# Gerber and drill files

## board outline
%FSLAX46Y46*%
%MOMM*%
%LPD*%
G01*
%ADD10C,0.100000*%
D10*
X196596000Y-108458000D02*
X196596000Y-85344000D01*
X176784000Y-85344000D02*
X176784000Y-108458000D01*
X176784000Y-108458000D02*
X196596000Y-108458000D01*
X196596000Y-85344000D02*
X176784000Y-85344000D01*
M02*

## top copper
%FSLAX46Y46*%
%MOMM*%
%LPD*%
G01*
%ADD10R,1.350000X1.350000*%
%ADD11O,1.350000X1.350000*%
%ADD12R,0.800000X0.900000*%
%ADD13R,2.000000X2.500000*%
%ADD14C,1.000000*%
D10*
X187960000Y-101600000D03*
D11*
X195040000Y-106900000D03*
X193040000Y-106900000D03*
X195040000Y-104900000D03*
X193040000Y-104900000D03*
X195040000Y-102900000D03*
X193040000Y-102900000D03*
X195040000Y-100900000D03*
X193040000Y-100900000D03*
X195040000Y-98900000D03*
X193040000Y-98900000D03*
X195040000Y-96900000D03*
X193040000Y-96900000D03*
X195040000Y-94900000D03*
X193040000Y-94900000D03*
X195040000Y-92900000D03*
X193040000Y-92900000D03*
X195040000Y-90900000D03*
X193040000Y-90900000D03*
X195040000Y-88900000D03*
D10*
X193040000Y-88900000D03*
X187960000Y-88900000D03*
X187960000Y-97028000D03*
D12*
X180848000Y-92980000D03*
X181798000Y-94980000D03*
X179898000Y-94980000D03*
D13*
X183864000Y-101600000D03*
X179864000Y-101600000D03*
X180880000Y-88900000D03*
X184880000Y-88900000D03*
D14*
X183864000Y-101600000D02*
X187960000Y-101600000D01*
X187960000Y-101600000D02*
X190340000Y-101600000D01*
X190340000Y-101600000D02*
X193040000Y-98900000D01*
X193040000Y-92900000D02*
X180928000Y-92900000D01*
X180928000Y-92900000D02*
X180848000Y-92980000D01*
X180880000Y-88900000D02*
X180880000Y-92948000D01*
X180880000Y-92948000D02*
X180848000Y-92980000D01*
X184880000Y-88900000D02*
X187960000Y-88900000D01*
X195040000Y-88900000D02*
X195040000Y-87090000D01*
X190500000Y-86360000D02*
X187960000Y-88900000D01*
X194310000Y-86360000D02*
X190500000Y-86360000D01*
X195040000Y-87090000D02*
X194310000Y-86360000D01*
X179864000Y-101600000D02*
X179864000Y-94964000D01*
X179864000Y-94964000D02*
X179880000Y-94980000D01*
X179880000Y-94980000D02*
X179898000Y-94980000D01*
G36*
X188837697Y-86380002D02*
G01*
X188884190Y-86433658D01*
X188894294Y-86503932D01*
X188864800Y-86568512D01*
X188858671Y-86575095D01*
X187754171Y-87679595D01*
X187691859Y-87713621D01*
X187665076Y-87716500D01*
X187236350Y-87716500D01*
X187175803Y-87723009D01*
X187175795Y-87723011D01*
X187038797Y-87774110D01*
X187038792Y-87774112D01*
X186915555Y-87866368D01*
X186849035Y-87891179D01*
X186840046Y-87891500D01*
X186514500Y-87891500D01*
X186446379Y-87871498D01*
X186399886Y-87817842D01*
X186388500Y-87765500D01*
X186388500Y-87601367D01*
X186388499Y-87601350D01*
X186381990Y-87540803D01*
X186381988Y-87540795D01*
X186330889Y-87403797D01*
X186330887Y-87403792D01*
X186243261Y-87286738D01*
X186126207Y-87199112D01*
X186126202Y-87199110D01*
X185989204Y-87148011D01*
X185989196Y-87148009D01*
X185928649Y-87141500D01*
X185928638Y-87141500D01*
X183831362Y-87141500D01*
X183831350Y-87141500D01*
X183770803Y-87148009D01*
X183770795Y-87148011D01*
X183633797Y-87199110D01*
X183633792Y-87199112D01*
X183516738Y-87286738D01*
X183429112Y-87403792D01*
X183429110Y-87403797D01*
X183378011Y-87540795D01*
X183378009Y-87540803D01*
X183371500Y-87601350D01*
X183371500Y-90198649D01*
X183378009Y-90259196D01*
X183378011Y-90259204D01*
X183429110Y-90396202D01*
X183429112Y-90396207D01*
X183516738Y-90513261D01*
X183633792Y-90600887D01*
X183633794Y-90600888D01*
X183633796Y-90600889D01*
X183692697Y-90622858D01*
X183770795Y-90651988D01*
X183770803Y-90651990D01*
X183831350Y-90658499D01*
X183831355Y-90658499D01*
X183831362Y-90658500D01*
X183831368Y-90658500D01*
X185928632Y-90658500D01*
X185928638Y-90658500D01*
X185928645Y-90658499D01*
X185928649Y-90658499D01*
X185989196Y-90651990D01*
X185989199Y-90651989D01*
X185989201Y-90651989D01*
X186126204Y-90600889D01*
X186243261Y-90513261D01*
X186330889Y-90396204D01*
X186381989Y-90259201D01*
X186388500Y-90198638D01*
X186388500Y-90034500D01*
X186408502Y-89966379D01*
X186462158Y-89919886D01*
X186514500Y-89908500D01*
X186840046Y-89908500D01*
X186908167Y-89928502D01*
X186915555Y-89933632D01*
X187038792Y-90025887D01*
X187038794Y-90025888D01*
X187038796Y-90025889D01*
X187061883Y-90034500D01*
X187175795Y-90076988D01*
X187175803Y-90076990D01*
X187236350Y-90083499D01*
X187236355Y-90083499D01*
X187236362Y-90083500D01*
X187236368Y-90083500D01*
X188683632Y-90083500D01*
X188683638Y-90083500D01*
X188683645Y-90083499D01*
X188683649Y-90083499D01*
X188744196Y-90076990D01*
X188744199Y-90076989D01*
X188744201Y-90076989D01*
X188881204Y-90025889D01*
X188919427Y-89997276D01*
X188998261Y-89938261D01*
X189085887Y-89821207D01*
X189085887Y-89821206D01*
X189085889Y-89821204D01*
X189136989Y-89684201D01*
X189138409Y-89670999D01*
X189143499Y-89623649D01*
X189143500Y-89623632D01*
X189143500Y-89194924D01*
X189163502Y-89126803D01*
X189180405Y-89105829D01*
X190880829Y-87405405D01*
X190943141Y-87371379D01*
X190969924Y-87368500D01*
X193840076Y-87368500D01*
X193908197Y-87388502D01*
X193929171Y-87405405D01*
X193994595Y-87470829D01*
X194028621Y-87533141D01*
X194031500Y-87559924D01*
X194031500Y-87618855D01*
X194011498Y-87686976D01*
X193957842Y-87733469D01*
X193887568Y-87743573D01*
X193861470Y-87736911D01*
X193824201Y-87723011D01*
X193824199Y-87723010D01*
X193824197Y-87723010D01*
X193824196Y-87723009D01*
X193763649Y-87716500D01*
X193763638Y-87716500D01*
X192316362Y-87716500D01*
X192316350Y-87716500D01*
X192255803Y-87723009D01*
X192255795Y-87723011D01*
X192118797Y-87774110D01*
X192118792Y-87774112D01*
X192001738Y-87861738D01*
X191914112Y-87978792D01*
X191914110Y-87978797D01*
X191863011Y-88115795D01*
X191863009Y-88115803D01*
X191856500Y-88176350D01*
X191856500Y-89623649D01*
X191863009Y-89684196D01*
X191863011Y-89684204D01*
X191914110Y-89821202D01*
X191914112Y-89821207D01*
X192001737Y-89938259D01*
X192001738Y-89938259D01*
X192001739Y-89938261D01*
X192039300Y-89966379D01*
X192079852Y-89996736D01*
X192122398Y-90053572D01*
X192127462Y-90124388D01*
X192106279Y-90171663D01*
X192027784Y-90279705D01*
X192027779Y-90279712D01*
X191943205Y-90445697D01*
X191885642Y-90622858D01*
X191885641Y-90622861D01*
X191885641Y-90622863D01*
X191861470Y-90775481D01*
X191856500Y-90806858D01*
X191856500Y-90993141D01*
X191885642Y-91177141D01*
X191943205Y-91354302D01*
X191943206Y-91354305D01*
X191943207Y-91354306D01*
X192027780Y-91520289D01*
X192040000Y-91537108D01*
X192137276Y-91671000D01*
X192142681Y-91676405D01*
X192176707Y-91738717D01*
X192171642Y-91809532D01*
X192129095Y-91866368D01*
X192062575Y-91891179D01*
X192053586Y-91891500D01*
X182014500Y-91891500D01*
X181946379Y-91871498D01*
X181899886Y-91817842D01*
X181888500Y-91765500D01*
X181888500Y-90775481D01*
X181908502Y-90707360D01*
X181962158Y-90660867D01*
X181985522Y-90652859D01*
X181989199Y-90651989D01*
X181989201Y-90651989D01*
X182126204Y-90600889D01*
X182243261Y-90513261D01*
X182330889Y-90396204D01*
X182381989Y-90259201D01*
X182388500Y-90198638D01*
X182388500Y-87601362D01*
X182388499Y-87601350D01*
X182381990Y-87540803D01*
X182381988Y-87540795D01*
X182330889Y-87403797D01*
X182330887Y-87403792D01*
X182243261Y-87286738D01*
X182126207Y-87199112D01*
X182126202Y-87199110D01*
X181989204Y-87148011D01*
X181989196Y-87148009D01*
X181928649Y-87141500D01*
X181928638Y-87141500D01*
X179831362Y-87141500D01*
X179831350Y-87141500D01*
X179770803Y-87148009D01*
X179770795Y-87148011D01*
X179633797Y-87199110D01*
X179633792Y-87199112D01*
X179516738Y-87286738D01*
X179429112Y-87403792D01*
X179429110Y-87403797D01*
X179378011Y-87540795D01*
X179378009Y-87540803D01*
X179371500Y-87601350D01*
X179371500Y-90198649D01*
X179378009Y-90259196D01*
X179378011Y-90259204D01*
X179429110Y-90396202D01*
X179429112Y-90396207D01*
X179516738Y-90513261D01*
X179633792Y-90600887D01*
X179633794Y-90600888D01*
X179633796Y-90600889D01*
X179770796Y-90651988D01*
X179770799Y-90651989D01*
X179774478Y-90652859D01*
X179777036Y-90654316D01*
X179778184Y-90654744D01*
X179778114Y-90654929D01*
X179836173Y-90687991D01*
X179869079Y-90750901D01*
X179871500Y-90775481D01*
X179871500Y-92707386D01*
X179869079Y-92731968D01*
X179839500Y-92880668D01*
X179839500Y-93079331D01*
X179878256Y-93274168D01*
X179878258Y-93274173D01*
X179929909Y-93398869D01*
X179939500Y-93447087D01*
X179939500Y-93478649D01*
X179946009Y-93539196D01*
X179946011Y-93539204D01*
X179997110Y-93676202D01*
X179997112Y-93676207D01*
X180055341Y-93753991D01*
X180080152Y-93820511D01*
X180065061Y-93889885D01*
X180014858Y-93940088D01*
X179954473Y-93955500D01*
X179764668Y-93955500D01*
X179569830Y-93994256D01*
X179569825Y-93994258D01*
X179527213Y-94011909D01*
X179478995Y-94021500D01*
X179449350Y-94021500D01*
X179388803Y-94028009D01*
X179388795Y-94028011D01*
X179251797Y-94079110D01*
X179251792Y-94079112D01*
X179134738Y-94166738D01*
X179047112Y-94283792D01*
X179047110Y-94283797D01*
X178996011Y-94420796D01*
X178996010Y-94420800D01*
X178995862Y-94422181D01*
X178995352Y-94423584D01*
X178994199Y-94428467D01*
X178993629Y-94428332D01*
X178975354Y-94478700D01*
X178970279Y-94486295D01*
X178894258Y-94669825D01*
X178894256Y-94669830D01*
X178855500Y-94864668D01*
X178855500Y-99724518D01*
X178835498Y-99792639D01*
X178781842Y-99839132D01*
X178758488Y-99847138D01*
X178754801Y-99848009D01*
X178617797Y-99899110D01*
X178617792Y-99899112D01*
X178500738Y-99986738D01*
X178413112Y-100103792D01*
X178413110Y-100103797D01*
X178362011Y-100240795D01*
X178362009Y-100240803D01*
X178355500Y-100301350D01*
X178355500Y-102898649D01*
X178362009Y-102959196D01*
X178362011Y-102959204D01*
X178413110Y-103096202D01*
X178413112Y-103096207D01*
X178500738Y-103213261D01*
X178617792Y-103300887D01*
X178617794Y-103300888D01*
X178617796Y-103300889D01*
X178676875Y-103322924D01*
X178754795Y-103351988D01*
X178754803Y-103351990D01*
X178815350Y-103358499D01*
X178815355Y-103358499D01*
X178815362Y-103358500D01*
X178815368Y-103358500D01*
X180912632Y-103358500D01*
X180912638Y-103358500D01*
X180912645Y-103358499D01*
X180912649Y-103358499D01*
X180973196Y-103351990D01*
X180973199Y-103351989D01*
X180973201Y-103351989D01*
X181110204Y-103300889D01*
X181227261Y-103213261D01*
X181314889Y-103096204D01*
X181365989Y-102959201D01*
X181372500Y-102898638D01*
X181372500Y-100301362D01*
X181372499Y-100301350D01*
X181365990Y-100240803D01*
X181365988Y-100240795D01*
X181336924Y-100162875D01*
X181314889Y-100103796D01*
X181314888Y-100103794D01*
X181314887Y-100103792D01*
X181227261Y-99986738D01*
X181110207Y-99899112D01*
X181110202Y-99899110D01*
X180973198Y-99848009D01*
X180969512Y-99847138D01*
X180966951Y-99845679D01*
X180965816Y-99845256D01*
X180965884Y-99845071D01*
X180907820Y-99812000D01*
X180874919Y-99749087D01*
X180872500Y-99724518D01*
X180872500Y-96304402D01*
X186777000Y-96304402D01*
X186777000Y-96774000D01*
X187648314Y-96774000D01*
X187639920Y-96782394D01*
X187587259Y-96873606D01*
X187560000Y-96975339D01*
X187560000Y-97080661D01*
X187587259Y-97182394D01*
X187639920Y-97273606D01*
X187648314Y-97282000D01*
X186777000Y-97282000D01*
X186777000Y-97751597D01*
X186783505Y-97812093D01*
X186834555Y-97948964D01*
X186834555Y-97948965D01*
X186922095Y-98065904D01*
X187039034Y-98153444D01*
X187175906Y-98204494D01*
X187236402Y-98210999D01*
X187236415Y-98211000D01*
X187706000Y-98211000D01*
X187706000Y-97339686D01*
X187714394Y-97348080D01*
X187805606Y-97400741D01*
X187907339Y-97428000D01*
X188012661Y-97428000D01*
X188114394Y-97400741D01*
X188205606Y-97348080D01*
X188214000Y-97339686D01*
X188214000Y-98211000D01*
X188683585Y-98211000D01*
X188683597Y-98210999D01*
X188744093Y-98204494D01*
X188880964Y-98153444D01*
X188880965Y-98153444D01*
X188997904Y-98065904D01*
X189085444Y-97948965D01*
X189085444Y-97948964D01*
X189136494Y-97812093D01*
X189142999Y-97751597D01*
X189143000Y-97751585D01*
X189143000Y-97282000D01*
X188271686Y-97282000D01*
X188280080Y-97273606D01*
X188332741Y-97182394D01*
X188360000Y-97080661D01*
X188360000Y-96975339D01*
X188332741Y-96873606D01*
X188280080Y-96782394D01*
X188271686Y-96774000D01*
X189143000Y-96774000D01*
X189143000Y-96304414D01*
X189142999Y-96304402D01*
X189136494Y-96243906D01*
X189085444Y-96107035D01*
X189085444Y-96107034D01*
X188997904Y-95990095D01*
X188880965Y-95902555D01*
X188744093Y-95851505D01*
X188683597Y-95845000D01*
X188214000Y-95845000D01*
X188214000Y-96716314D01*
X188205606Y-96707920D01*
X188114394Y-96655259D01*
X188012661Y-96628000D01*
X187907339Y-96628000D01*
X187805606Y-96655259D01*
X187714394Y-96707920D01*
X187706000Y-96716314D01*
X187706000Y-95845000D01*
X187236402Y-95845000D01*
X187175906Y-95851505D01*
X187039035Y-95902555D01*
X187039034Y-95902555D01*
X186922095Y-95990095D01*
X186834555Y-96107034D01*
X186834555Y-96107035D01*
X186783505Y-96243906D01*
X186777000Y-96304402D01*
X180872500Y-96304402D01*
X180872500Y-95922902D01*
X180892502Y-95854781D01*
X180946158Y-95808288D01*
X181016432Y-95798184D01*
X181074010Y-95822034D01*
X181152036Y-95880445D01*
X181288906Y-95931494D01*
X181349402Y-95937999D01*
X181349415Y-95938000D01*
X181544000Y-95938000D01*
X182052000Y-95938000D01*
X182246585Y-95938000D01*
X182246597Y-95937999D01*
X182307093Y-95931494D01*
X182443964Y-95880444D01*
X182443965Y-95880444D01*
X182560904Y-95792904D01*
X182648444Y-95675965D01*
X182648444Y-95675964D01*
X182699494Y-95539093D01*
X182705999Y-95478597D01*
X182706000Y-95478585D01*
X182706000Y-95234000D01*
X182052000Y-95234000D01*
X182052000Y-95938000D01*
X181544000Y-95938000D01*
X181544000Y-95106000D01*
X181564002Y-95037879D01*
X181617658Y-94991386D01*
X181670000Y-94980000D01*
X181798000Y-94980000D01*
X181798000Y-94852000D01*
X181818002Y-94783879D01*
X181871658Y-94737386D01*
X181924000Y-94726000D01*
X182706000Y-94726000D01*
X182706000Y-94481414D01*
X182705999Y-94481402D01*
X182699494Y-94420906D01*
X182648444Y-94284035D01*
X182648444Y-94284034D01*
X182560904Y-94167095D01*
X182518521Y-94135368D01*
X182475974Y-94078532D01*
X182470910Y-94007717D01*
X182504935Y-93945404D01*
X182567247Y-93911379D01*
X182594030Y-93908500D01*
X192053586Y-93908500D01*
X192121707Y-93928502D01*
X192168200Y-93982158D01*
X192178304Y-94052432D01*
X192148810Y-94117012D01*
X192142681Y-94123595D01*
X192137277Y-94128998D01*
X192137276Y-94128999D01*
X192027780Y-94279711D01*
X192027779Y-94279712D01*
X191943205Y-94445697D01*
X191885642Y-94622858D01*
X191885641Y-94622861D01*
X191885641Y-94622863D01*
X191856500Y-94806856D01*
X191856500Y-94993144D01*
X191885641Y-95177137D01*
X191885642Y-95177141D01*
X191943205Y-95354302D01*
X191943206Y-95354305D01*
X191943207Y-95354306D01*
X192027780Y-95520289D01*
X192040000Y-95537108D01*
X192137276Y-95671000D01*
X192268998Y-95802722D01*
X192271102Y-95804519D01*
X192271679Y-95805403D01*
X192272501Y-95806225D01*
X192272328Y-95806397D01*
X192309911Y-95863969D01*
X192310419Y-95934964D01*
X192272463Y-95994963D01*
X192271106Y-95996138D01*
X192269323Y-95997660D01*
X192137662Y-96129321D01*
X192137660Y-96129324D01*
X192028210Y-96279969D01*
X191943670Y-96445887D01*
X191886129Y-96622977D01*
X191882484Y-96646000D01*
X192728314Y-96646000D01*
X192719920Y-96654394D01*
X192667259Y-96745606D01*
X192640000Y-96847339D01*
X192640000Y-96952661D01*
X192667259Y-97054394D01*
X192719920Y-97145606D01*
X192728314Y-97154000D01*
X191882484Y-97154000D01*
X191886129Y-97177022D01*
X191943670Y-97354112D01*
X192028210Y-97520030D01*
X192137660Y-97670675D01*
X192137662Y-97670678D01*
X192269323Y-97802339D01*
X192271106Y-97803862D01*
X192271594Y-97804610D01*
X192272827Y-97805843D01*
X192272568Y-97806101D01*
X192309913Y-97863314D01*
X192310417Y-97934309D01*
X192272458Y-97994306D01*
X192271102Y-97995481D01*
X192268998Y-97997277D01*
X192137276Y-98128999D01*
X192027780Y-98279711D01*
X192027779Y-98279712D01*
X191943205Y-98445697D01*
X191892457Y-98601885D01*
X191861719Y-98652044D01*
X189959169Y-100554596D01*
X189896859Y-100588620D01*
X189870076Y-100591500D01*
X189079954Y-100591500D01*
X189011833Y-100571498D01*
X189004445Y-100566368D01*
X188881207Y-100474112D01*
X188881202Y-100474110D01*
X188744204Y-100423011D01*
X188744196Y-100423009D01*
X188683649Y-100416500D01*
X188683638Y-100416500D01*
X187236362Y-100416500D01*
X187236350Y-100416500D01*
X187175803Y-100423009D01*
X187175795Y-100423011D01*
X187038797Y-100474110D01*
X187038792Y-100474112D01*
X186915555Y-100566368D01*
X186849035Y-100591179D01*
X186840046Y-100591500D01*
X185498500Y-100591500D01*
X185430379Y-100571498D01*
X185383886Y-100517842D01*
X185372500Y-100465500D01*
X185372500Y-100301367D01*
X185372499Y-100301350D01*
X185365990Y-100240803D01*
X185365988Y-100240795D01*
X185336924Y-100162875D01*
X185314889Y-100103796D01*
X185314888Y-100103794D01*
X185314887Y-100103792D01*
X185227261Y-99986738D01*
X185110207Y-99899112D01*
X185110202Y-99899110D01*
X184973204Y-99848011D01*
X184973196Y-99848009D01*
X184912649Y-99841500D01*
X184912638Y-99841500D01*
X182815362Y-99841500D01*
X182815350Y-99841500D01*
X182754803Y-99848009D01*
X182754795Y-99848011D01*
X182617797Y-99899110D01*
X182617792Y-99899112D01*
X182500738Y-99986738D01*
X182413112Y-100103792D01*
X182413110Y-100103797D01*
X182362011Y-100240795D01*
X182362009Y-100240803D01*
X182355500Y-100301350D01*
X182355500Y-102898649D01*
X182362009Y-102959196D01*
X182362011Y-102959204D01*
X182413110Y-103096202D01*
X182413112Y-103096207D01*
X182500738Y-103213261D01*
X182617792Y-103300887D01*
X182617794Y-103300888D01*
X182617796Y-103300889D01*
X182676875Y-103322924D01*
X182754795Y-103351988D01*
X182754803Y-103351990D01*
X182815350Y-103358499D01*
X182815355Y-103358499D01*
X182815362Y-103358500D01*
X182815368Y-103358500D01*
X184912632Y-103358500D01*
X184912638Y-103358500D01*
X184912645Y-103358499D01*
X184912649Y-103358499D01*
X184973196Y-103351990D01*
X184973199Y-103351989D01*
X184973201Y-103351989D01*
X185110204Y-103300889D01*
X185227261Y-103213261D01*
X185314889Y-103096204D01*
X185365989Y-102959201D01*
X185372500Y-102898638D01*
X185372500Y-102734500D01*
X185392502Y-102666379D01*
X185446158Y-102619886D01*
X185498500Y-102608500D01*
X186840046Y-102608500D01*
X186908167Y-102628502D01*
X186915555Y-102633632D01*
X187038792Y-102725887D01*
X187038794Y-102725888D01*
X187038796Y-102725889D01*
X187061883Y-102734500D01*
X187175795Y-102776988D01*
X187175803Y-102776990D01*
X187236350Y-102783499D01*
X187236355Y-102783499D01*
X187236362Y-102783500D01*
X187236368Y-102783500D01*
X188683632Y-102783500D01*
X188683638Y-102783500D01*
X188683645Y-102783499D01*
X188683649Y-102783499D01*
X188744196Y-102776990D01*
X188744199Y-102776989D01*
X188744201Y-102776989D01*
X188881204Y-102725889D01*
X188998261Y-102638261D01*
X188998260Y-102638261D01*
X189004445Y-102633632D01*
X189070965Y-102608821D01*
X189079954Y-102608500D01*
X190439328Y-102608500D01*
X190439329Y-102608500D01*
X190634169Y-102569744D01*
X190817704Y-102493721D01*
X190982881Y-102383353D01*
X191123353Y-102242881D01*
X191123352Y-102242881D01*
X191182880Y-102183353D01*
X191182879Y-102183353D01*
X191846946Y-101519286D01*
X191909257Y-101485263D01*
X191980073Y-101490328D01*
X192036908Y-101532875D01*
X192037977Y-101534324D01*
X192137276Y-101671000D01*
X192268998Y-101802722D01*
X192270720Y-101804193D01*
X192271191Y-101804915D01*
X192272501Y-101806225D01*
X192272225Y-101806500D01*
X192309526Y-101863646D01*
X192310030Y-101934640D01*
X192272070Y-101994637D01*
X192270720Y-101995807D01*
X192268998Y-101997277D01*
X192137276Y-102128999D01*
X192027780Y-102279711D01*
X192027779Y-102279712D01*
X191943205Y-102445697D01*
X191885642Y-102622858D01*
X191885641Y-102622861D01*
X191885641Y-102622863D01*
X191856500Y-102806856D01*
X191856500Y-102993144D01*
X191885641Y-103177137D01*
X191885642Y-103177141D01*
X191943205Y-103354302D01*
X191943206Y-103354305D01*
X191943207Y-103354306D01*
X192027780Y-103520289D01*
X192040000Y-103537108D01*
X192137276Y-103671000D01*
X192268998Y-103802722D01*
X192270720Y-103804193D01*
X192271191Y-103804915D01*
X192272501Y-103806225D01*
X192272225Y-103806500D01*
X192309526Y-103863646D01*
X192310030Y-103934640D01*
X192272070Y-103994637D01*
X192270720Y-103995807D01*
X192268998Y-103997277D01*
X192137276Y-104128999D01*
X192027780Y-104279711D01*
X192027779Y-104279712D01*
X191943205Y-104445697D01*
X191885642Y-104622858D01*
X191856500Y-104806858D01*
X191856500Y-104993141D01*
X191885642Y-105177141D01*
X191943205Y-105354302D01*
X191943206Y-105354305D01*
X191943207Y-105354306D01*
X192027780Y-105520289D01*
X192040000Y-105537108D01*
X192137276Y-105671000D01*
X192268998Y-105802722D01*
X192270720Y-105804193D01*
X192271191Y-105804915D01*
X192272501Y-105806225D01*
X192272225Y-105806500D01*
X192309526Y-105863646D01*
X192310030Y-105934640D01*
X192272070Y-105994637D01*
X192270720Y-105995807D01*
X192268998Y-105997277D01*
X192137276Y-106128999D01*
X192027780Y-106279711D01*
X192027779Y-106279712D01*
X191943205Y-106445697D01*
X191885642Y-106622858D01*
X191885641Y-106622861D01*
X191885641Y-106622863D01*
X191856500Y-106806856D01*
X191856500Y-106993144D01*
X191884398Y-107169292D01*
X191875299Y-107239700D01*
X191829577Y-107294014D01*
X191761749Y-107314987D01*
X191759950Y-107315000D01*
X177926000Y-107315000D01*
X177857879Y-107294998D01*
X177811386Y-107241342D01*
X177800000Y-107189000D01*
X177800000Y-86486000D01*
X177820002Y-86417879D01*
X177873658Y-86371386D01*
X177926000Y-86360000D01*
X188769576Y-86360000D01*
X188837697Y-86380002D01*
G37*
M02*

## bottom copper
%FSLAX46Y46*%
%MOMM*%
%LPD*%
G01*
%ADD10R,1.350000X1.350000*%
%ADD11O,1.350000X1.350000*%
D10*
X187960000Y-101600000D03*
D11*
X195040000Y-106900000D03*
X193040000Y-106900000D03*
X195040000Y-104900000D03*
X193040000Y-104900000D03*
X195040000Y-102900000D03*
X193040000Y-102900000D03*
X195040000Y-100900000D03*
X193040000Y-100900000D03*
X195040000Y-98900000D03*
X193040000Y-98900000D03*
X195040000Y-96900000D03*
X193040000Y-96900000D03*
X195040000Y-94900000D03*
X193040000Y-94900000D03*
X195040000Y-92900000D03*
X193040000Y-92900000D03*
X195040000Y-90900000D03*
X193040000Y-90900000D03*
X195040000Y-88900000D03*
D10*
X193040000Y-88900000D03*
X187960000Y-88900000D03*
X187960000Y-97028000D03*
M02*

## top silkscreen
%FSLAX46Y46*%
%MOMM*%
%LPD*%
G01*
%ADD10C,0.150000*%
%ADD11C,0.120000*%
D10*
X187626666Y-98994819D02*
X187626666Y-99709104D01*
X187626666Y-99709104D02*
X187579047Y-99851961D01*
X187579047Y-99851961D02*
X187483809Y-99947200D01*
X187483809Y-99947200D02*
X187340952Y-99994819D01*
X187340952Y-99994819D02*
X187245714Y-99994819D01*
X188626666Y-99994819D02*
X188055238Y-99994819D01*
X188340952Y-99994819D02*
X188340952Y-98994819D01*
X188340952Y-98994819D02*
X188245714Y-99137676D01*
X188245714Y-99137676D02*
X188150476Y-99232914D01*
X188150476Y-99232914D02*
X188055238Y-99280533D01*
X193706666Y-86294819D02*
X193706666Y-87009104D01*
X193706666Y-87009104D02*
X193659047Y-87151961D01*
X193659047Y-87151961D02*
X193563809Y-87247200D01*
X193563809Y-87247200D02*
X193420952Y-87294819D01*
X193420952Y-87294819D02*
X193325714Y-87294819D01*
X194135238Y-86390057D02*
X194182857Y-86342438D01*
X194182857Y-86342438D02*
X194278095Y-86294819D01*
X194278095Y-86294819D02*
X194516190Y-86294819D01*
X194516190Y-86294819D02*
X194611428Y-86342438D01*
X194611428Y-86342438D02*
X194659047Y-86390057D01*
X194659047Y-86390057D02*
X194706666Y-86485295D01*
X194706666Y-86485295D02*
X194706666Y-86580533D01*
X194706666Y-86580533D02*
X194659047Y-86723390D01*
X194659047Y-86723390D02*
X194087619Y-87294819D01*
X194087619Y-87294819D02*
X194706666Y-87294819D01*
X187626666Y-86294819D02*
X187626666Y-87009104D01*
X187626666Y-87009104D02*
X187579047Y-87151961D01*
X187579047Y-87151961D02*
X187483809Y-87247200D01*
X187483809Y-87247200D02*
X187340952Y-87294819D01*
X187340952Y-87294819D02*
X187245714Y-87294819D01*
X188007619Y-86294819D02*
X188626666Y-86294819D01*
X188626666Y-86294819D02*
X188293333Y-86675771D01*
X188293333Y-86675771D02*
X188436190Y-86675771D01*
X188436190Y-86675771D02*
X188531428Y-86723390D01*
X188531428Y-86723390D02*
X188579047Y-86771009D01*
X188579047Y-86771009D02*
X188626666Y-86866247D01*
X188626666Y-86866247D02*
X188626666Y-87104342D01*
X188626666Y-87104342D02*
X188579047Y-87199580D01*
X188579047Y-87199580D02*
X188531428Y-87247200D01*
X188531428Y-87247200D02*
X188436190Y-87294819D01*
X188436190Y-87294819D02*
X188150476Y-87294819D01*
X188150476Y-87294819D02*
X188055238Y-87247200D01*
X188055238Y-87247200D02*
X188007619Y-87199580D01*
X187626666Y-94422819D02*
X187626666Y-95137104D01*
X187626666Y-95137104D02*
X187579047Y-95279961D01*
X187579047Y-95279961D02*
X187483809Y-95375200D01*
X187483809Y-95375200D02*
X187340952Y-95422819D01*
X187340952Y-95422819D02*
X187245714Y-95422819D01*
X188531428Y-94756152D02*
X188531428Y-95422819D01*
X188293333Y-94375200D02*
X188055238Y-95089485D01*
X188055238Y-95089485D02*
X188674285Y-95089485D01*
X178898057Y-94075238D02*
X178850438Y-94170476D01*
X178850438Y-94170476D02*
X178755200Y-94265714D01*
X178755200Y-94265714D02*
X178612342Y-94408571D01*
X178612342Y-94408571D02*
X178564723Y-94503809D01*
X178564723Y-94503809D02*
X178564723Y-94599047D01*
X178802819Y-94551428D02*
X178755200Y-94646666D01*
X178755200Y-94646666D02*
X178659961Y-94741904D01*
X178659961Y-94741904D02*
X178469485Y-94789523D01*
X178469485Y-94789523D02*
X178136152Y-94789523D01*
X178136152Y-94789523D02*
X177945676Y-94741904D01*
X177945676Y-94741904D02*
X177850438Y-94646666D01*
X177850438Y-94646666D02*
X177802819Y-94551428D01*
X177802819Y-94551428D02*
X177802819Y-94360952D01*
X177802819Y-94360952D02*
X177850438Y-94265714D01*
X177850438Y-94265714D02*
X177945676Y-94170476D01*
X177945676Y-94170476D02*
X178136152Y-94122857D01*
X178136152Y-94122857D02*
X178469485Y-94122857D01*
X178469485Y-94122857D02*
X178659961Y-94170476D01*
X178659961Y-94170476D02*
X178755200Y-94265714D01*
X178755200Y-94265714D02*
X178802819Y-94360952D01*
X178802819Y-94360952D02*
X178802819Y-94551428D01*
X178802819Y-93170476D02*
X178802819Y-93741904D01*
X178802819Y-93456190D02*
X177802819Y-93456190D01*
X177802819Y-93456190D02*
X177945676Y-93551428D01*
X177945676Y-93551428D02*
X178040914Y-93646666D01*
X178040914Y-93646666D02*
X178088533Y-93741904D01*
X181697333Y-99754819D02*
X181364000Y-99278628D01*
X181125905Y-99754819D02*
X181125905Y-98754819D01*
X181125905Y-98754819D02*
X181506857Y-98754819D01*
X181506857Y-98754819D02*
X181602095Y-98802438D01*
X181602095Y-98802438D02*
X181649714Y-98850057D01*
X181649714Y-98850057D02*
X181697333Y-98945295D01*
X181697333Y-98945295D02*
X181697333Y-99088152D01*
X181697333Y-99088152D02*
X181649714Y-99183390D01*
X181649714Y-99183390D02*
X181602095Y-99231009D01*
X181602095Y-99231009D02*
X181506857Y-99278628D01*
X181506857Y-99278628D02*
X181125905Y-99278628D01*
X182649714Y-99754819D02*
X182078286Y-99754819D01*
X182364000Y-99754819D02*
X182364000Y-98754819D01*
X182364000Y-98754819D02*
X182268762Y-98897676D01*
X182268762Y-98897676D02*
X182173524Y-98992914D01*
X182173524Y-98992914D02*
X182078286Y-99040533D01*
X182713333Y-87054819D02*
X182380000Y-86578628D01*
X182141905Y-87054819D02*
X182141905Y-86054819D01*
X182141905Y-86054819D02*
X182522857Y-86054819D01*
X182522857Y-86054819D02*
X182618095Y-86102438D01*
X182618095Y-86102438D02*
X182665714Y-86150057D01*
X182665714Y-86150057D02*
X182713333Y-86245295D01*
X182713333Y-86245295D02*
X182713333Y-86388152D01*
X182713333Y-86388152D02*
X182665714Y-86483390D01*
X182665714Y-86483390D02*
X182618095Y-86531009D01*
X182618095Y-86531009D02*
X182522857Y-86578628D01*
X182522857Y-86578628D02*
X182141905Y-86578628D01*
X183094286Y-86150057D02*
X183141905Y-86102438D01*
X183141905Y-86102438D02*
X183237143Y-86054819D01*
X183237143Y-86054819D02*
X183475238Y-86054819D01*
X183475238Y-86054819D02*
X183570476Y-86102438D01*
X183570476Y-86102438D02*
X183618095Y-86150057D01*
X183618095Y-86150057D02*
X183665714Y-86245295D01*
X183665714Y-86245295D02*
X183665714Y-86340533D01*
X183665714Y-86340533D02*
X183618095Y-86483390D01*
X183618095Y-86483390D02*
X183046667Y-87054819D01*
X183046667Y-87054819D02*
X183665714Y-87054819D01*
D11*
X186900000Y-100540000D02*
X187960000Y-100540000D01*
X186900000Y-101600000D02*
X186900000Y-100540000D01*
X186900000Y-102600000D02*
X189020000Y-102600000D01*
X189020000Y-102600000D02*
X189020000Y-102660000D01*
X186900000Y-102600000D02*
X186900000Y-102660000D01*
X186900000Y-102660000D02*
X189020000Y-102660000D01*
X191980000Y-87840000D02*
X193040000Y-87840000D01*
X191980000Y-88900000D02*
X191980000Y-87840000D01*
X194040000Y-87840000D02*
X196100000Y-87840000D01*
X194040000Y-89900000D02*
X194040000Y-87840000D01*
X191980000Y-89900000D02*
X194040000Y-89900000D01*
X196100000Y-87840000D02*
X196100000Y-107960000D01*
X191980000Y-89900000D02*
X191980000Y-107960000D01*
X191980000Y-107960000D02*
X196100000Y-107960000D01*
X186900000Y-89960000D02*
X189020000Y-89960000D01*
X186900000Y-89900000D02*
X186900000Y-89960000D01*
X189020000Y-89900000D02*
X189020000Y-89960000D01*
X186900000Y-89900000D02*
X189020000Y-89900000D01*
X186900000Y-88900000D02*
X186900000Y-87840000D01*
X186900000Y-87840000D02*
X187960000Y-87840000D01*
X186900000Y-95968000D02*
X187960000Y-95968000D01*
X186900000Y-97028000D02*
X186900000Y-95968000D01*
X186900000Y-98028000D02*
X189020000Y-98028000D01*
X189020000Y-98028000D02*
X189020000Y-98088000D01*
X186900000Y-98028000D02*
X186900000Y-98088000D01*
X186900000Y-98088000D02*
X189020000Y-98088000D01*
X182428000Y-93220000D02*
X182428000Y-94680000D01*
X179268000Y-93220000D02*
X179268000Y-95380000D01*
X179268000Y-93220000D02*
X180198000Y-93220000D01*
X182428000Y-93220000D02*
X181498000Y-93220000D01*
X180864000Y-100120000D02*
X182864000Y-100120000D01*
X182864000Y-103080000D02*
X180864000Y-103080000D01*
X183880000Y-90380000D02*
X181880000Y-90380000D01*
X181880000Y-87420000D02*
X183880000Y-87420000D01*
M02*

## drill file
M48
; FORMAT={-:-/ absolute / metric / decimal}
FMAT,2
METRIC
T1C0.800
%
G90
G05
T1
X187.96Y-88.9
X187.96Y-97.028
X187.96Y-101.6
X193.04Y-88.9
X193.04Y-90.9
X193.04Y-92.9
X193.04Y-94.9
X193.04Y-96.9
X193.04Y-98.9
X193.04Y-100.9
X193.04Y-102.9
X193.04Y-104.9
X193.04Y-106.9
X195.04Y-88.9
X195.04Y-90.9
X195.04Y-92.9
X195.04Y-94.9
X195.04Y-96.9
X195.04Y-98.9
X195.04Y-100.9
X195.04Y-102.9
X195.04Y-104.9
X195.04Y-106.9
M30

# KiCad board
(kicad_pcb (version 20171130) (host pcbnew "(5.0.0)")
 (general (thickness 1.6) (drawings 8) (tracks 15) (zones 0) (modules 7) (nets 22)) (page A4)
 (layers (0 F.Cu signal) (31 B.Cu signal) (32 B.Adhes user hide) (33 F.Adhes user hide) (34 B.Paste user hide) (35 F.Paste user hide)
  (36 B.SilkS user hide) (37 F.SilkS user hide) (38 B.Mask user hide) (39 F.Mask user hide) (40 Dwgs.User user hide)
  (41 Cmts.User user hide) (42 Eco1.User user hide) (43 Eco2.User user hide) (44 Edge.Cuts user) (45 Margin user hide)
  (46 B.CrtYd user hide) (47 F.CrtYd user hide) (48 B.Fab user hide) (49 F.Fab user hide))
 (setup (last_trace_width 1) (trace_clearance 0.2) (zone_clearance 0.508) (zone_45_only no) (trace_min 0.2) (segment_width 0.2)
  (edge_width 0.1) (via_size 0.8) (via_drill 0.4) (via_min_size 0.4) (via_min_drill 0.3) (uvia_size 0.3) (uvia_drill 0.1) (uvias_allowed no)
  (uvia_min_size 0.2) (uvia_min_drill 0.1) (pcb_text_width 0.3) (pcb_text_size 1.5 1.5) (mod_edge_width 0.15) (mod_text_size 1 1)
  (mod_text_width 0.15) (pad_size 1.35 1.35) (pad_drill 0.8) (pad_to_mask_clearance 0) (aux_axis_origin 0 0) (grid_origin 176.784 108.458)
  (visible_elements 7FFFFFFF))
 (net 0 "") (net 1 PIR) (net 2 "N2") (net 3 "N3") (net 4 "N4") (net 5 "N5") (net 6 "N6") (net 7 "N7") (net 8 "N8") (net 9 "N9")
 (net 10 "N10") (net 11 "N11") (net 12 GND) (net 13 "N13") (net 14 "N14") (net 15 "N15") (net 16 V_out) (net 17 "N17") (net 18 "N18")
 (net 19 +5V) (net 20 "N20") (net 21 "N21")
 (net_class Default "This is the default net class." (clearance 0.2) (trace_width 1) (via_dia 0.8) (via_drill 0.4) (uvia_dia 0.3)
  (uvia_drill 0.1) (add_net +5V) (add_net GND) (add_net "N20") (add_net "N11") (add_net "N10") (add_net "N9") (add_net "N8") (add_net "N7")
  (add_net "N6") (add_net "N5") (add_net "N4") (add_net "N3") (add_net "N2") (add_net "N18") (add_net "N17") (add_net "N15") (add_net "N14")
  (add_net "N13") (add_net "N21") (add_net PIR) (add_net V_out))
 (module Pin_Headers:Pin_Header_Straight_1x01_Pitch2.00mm (layer F.Cu) (at 187.96 101.6)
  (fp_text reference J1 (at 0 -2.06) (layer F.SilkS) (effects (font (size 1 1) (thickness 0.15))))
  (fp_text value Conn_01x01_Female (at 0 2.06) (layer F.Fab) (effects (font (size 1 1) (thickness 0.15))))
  (fp_line (start -1.06 -1.06) (end 0 -1.06) (layer F.SilkS) (width 0.12))
  (fp_line (start -1.06 0) (end -1.06 -1.06) (layer F.SilkS) (width 0.12))
  (fp_line (start -1.06 1) (end 1.06 1) (layer F.SilkS) (width 0.12))
  (fp_line (start 1.06 1) (end 1.06 1.06) (layer F.SilkS) (width 0.12))
  (fp_line (start -1.06 1) (end -1.06 1.06) (layer F.SilkS) (width 0.12))
  (fp_line (start -1.06 1.06) (end 1.06 1.06) (layer F.SilkS) (width 0.12))
  (pad 1 thru_hole rect (at 0 0) (size 1.35 1.35) (drill 0.8) (layers *.Cu *.Mask) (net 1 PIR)))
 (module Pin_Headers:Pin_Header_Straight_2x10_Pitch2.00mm (layer F.Cu) (at 193.04 88.9)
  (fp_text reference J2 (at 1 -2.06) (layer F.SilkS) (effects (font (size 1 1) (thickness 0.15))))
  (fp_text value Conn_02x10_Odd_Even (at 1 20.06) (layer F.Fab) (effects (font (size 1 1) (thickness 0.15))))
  (fp_line (start -1.06 -1.06) (end 0 -1.06) (layer F.SilkS) (width 0.12))
  (fp_line (start -1.06 0) (end -1.06 -1.06) (layer F.SilkS) (width 0.12))
  (fp_line (start 1 -1.06) (end 3.06 -1.06) (layer F.SilkS) (width 0.12))
  (fp_line (start 1 1) (end 1 -1.06) (layer F.SilkS) (width 0.12))
  (fp_line (start -1.06 1) (end 1 1) (layer F.SilkS) (width 0.12))
  (fp_line (start 3.06 -1.06) (end 3.06 19.06) (layer F.SilkS) (width 0.12))
  (fp_line (start -1.06 1) (end -1.06 19.06) (layer F.SilkS) (width 0.12))
  (fp_line (start -1.06 19.06) (end 3.06 19.06) (layer F.SilkS) (width 0.12))
  (pad 20 thru_hole oval (at 2 18) (size 1.35 1.35) (drill 0.8) (layers *.Cu *.Mask) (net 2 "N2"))
  (pad 19 thru_hole oval (at 0 18) (size 1.35 1.35) (drill 0.8) (layers *.Cu *.Mask) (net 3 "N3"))
  (pad 18 thru_hole oval (at 2 16) (size 1.35 1.35) (drill 0.8) (layers *.Cu *.Mask) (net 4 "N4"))
  (pad 17 thru_hole oval (at 0 16) (size 1.35 1.35) (drill 0.8) (layers *.Cu *.Mask) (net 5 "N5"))
  (pad 16 thru_hole oval (at 2 14) (size 1.35 1.35) (drill 0.8) (layers *.Cu *.Mask) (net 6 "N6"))
  (pad 15 thru_hole oval (at 0 14) (size 1.35 1.35) (drill 0.8) (layers *.Cu *.Mask) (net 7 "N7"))
  (pad 14 thru_hole oval (at 2 12) (size 1.35 1.35) (drill 0.8) (layers *.Cu *.Mask) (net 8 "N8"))
  (pad 13 thru_hole oval (at 0 12) (size 1.35 1.35) (drill 0.8) (layers *.Cu *.Mask) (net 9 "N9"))
  (pad 12 thru_hole oval (at 2 10) (size 1.35 1.35) (drill 0.8) (layers *.Cu *.Mask) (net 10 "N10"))
  (pad 11 thru_hole oval (at 0 10) (size 1.35 1.35) (drill 0.8) (layers *.Cu *.Mask) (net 1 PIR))
  (pad 10 thru_hole oval (at 2 8) (size 1.35 1.35) (drill 0.8) (layers *.Cu *.Mask) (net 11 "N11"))
  (pad 9 thru_hole oval (at 0 8) (size 1.35 1.35) (drill 0.8) (layers *.Cu *.Mask) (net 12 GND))
  (pad 8 thru_hole oval (at 2 6) (size 1.35 1.35) (drill 0.8) (layers *.Cu *.Mask) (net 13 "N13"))
  (pad 7 thru_hole oval (at 0 6) (size 1.35 1.35) (drill 0.8) (layers *.Cu *.Mask) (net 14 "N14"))
  (pad 6 thru_hole oval (at 2 4) (size 1.35 1.35) (drill 0.8) (layers *.Cu *.Mask) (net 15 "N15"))
  (pad 5 thru_hole oval (at 0 4) (size 1.35 1.35) (drill 0.8) (layers *.Cu *.Mask) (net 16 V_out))
  (pad 4 thru_hole oval (at 2 2) (size 1.35 1.35) (drill 0.8) (layers *.Cu *.Mask) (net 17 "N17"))
  (pad 3 thru_hole oval (at 0 2) (size 1.35 1.35) (drill 0.8) (layers *.Cu *.Mask) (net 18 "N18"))
  (pad 2 thru_hole oval (at 2 0) (size 1.35 1.35) (drill 0.8) (layers *.Cu *.Mask) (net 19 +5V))
  (pad 1 thru_hole rect (at 0 0) (size 1.35 1.35) (drill 0.8) (layers *.Cu *.Mask) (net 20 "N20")))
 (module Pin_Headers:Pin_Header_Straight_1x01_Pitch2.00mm (layer F.Cu) (at 187.96 88.9)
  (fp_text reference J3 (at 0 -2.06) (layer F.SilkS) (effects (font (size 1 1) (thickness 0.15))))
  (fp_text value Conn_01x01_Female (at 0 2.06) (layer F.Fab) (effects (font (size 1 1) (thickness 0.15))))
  (fp_line (start -1.06 1.06) (end 1.06 1.06) (layer F.SilkS) (width 0.12))
  (fp_line (start -1.06 1) (end -1.06 1.06) (layer F.SilkS) (width 0.12))
  (fp_line (start 1.06 1) (end 1.06 1.06) (layer F.SilkS) (width 0.12))
  (fp_line (start -1.06 1) (end 1.06 1) (layer F.SilkS) (width 0.12))
  (fp_line (start -1.06 0) (end -1.06 -1.06) (layer F.SilkS) (width 0.12))
  (fp_line (start -1.06 -1.06) (end 0 -1.06) (layer F.SilkS) (width 0.12))
  (pad 1 thru_hole rect (at 0 0) (size 1.35 1.35) (drill 0.8) (layers *.Cu *.Mask) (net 19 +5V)))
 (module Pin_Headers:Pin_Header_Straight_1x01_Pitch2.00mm (layer F.Cu) (at 187.96 97.028)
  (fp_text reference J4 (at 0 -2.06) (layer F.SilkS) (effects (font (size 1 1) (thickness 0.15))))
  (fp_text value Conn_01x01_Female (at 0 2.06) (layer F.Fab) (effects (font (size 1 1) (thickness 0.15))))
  (fp_line (start -1.06 -1.06) (end 0 -1.06) (layer F.SilkS) (width 0.12))
  (fp_line (start -1.06 0) (end -1.06 -1.06) (layer F.SilkS) (width 0.12))
  (fp_line (start -1.06 1) (end 1.06 1) (layer F.SilkS) (width 0.12))
  (fp_line (start 1.06 1) (end 1.06 1.06) (layer F.SilkS) (width 0.12))
  (fp_line (start -1.06 1) (end -1.06 1.06) (layer F.SilkS) (width 0.12))
  (fp_line (start -1.06 1.06) (end 1.06 1.06) (layer F.SilkS) (width 0.12))
  (pad 1 thru_hole rect (at 0 0) (size 1.35 1.35) (drill 0.8) (layers *.Cu *.Mask) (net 12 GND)))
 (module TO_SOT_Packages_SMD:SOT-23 (layer F.Cu) (at 180.848 93.98 90)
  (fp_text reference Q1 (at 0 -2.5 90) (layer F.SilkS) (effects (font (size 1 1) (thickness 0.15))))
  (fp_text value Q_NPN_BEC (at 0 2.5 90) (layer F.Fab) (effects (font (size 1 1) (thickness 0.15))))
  (fp_line (start 0.76 1.58) (end -0.7 1.58) (layer F.SilkS) (width 0.12))
  (fp_line (start 0.76 -1.58) (end -1.4 -1.58) (layer F.SilkS) (width 0.12))
  (fp_line (start 0.76 -1.58) (end 0.76 -0.65) (layer F.SilkS) (width 0.12))
  (fp_line (start 0.76 1.58) (end 0.76 0.65) (layer F.SilkS) (width 0.12))
  (pad 3 smd rect (at 1 0 90) (size 0.9 0.8) (layers F.Cu F.Paste F.Mask) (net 16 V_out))
  (pad 2 smd rect (at -1 0.95 90) (size 0.9 0.8) (layers F.Cu F.Paste F.Mask) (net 12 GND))
  (pad 1 smd rect (at -1 -0.95 90) (size 0.9 0.8) (layers F.Cu F.Paste F.Mask) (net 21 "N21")))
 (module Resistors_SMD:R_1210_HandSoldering (layer F.Cu) (at 181.864 101.6)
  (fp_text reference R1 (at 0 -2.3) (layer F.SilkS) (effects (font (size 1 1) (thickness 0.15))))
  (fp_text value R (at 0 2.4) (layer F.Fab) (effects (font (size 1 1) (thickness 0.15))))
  (fp_line (start -1 -1.48) (end 1 -1.48) (layer F.SilkS) (width 0.12))
  (fp_line (start 1 1.48) (end -1 1.48) (layer F.SilkS) (width 0.12))
  (pad 2 smd rect (at 2 0) (size 2 2.5) (layers F.Cu F.Paste F.Mask) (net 1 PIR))
  (pad 1 smd rect (at -2 0) (size 2 2.5) (layers F.Cu F.Paste F.Mask) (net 21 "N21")))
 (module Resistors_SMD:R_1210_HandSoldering (layer F.Cu) (at 182.88 88.9)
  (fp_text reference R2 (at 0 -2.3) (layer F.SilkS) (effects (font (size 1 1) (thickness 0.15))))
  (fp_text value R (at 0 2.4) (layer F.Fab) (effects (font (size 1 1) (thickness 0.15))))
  (fp_line (start 1 1.48) (end -1 1.48) (layer F.SilkS) (width 0.12))
  (fp_line (start -1 -1.48) (end 1 -1.48) (layer F.SilkS) (width 0.12))
  (pad 1 smd rect (at -2 0) (size 2 2.5) (layers F.Cu F.Paste F.Mask) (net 16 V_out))
  (pad 2 smd rect (at 2 0) (size 2 2.5) (layers F.Cu F.Paste F.Mask) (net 19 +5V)))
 (gr_line (start 196.596 108.458) (end 196.596 85.344) (angle 90) (layer Edge.Cuts) (width 0.1))
 (gr_line (start 176.784 85.344) (end 176.784 108.458) (angle 90) (layer Edge.Cuts) (width 0.1))
 (gr_line (start 176.784 108.458) (end 196.596 108.458) (angle 90) (layer Edge.Cuts) (width 0.1))
 (gr_line (start 196.596 85.344) (end 176.784 85.344) (angle 90) (layer Edge.Cuts) (width 0.1))
 (segment (start 183.864 101.6) (end 187.96 101.6) (width 1) (layer F.Cu) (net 1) (status C00000))
 (segment (start 187.96 101.6) (end 190.34 101.6) (width 1) (layer F.Cu) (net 1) (status 400000))
 (segment (start 190.34 101.6) (end 193.04 98.9) (width 1) (layer F.Cu) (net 1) (status 800000))
 (segment (start 193.04 92.9) (end 180.928 92.9) (width 1) (layer F.Cu) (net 16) (status C00000))
 (segment (start 180.928 92.9) (end 180.848 92.98) (width 1) (layer F.Cu) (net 16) (status C00000))
 (segment (start 180.88 88.9) (end 180.88 92.948) (width 1) (layer F.Cu) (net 16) (status C00000))
 (segment (start 180.88 92.948) (end 180.848 92.98) (width 1) (layer F.Cu) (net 16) (status C00000))
 (segment (start 184.88 88.9) (end 187.96 88.9) (width 1) (layer F.Cu) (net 19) (status C00000))
 (segment (start 195.04 88.9) (end 195.04 87.09) (width 1) (layer F.Cu) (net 19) (status 400000))
 (segment (start 190.5 86.36) (end 187.96 88.9) (width 1) (layer F.Cu) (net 19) (status 800000))
 (segment (start 194.31 86.36) (end 190.5 86.36) (width 1) (layer F.Cu) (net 19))
 (segment (start 195.04 87.09) (end 194.31 86.36) (width 1) (layer F.Cu) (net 19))
 (segment (start 179.864 101.6) (end 179.864 94.964) (width 1) (layer F.Cu) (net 21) (status C00000))
 (segment (start 179.864 94.964) (end 179.88 94.98) (width 1) (layer F.Cu) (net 21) (status C00000))
 (segment (start 179.88 94.98) (end 179.898 94.98) (width 1) (layer F.Cu) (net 21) (status C00000))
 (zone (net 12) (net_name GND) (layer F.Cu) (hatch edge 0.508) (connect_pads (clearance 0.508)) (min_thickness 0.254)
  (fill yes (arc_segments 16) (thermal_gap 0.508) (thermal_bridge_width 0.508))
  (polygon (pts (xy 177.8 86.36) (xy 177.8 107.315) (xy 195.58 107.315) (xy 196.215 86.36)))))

